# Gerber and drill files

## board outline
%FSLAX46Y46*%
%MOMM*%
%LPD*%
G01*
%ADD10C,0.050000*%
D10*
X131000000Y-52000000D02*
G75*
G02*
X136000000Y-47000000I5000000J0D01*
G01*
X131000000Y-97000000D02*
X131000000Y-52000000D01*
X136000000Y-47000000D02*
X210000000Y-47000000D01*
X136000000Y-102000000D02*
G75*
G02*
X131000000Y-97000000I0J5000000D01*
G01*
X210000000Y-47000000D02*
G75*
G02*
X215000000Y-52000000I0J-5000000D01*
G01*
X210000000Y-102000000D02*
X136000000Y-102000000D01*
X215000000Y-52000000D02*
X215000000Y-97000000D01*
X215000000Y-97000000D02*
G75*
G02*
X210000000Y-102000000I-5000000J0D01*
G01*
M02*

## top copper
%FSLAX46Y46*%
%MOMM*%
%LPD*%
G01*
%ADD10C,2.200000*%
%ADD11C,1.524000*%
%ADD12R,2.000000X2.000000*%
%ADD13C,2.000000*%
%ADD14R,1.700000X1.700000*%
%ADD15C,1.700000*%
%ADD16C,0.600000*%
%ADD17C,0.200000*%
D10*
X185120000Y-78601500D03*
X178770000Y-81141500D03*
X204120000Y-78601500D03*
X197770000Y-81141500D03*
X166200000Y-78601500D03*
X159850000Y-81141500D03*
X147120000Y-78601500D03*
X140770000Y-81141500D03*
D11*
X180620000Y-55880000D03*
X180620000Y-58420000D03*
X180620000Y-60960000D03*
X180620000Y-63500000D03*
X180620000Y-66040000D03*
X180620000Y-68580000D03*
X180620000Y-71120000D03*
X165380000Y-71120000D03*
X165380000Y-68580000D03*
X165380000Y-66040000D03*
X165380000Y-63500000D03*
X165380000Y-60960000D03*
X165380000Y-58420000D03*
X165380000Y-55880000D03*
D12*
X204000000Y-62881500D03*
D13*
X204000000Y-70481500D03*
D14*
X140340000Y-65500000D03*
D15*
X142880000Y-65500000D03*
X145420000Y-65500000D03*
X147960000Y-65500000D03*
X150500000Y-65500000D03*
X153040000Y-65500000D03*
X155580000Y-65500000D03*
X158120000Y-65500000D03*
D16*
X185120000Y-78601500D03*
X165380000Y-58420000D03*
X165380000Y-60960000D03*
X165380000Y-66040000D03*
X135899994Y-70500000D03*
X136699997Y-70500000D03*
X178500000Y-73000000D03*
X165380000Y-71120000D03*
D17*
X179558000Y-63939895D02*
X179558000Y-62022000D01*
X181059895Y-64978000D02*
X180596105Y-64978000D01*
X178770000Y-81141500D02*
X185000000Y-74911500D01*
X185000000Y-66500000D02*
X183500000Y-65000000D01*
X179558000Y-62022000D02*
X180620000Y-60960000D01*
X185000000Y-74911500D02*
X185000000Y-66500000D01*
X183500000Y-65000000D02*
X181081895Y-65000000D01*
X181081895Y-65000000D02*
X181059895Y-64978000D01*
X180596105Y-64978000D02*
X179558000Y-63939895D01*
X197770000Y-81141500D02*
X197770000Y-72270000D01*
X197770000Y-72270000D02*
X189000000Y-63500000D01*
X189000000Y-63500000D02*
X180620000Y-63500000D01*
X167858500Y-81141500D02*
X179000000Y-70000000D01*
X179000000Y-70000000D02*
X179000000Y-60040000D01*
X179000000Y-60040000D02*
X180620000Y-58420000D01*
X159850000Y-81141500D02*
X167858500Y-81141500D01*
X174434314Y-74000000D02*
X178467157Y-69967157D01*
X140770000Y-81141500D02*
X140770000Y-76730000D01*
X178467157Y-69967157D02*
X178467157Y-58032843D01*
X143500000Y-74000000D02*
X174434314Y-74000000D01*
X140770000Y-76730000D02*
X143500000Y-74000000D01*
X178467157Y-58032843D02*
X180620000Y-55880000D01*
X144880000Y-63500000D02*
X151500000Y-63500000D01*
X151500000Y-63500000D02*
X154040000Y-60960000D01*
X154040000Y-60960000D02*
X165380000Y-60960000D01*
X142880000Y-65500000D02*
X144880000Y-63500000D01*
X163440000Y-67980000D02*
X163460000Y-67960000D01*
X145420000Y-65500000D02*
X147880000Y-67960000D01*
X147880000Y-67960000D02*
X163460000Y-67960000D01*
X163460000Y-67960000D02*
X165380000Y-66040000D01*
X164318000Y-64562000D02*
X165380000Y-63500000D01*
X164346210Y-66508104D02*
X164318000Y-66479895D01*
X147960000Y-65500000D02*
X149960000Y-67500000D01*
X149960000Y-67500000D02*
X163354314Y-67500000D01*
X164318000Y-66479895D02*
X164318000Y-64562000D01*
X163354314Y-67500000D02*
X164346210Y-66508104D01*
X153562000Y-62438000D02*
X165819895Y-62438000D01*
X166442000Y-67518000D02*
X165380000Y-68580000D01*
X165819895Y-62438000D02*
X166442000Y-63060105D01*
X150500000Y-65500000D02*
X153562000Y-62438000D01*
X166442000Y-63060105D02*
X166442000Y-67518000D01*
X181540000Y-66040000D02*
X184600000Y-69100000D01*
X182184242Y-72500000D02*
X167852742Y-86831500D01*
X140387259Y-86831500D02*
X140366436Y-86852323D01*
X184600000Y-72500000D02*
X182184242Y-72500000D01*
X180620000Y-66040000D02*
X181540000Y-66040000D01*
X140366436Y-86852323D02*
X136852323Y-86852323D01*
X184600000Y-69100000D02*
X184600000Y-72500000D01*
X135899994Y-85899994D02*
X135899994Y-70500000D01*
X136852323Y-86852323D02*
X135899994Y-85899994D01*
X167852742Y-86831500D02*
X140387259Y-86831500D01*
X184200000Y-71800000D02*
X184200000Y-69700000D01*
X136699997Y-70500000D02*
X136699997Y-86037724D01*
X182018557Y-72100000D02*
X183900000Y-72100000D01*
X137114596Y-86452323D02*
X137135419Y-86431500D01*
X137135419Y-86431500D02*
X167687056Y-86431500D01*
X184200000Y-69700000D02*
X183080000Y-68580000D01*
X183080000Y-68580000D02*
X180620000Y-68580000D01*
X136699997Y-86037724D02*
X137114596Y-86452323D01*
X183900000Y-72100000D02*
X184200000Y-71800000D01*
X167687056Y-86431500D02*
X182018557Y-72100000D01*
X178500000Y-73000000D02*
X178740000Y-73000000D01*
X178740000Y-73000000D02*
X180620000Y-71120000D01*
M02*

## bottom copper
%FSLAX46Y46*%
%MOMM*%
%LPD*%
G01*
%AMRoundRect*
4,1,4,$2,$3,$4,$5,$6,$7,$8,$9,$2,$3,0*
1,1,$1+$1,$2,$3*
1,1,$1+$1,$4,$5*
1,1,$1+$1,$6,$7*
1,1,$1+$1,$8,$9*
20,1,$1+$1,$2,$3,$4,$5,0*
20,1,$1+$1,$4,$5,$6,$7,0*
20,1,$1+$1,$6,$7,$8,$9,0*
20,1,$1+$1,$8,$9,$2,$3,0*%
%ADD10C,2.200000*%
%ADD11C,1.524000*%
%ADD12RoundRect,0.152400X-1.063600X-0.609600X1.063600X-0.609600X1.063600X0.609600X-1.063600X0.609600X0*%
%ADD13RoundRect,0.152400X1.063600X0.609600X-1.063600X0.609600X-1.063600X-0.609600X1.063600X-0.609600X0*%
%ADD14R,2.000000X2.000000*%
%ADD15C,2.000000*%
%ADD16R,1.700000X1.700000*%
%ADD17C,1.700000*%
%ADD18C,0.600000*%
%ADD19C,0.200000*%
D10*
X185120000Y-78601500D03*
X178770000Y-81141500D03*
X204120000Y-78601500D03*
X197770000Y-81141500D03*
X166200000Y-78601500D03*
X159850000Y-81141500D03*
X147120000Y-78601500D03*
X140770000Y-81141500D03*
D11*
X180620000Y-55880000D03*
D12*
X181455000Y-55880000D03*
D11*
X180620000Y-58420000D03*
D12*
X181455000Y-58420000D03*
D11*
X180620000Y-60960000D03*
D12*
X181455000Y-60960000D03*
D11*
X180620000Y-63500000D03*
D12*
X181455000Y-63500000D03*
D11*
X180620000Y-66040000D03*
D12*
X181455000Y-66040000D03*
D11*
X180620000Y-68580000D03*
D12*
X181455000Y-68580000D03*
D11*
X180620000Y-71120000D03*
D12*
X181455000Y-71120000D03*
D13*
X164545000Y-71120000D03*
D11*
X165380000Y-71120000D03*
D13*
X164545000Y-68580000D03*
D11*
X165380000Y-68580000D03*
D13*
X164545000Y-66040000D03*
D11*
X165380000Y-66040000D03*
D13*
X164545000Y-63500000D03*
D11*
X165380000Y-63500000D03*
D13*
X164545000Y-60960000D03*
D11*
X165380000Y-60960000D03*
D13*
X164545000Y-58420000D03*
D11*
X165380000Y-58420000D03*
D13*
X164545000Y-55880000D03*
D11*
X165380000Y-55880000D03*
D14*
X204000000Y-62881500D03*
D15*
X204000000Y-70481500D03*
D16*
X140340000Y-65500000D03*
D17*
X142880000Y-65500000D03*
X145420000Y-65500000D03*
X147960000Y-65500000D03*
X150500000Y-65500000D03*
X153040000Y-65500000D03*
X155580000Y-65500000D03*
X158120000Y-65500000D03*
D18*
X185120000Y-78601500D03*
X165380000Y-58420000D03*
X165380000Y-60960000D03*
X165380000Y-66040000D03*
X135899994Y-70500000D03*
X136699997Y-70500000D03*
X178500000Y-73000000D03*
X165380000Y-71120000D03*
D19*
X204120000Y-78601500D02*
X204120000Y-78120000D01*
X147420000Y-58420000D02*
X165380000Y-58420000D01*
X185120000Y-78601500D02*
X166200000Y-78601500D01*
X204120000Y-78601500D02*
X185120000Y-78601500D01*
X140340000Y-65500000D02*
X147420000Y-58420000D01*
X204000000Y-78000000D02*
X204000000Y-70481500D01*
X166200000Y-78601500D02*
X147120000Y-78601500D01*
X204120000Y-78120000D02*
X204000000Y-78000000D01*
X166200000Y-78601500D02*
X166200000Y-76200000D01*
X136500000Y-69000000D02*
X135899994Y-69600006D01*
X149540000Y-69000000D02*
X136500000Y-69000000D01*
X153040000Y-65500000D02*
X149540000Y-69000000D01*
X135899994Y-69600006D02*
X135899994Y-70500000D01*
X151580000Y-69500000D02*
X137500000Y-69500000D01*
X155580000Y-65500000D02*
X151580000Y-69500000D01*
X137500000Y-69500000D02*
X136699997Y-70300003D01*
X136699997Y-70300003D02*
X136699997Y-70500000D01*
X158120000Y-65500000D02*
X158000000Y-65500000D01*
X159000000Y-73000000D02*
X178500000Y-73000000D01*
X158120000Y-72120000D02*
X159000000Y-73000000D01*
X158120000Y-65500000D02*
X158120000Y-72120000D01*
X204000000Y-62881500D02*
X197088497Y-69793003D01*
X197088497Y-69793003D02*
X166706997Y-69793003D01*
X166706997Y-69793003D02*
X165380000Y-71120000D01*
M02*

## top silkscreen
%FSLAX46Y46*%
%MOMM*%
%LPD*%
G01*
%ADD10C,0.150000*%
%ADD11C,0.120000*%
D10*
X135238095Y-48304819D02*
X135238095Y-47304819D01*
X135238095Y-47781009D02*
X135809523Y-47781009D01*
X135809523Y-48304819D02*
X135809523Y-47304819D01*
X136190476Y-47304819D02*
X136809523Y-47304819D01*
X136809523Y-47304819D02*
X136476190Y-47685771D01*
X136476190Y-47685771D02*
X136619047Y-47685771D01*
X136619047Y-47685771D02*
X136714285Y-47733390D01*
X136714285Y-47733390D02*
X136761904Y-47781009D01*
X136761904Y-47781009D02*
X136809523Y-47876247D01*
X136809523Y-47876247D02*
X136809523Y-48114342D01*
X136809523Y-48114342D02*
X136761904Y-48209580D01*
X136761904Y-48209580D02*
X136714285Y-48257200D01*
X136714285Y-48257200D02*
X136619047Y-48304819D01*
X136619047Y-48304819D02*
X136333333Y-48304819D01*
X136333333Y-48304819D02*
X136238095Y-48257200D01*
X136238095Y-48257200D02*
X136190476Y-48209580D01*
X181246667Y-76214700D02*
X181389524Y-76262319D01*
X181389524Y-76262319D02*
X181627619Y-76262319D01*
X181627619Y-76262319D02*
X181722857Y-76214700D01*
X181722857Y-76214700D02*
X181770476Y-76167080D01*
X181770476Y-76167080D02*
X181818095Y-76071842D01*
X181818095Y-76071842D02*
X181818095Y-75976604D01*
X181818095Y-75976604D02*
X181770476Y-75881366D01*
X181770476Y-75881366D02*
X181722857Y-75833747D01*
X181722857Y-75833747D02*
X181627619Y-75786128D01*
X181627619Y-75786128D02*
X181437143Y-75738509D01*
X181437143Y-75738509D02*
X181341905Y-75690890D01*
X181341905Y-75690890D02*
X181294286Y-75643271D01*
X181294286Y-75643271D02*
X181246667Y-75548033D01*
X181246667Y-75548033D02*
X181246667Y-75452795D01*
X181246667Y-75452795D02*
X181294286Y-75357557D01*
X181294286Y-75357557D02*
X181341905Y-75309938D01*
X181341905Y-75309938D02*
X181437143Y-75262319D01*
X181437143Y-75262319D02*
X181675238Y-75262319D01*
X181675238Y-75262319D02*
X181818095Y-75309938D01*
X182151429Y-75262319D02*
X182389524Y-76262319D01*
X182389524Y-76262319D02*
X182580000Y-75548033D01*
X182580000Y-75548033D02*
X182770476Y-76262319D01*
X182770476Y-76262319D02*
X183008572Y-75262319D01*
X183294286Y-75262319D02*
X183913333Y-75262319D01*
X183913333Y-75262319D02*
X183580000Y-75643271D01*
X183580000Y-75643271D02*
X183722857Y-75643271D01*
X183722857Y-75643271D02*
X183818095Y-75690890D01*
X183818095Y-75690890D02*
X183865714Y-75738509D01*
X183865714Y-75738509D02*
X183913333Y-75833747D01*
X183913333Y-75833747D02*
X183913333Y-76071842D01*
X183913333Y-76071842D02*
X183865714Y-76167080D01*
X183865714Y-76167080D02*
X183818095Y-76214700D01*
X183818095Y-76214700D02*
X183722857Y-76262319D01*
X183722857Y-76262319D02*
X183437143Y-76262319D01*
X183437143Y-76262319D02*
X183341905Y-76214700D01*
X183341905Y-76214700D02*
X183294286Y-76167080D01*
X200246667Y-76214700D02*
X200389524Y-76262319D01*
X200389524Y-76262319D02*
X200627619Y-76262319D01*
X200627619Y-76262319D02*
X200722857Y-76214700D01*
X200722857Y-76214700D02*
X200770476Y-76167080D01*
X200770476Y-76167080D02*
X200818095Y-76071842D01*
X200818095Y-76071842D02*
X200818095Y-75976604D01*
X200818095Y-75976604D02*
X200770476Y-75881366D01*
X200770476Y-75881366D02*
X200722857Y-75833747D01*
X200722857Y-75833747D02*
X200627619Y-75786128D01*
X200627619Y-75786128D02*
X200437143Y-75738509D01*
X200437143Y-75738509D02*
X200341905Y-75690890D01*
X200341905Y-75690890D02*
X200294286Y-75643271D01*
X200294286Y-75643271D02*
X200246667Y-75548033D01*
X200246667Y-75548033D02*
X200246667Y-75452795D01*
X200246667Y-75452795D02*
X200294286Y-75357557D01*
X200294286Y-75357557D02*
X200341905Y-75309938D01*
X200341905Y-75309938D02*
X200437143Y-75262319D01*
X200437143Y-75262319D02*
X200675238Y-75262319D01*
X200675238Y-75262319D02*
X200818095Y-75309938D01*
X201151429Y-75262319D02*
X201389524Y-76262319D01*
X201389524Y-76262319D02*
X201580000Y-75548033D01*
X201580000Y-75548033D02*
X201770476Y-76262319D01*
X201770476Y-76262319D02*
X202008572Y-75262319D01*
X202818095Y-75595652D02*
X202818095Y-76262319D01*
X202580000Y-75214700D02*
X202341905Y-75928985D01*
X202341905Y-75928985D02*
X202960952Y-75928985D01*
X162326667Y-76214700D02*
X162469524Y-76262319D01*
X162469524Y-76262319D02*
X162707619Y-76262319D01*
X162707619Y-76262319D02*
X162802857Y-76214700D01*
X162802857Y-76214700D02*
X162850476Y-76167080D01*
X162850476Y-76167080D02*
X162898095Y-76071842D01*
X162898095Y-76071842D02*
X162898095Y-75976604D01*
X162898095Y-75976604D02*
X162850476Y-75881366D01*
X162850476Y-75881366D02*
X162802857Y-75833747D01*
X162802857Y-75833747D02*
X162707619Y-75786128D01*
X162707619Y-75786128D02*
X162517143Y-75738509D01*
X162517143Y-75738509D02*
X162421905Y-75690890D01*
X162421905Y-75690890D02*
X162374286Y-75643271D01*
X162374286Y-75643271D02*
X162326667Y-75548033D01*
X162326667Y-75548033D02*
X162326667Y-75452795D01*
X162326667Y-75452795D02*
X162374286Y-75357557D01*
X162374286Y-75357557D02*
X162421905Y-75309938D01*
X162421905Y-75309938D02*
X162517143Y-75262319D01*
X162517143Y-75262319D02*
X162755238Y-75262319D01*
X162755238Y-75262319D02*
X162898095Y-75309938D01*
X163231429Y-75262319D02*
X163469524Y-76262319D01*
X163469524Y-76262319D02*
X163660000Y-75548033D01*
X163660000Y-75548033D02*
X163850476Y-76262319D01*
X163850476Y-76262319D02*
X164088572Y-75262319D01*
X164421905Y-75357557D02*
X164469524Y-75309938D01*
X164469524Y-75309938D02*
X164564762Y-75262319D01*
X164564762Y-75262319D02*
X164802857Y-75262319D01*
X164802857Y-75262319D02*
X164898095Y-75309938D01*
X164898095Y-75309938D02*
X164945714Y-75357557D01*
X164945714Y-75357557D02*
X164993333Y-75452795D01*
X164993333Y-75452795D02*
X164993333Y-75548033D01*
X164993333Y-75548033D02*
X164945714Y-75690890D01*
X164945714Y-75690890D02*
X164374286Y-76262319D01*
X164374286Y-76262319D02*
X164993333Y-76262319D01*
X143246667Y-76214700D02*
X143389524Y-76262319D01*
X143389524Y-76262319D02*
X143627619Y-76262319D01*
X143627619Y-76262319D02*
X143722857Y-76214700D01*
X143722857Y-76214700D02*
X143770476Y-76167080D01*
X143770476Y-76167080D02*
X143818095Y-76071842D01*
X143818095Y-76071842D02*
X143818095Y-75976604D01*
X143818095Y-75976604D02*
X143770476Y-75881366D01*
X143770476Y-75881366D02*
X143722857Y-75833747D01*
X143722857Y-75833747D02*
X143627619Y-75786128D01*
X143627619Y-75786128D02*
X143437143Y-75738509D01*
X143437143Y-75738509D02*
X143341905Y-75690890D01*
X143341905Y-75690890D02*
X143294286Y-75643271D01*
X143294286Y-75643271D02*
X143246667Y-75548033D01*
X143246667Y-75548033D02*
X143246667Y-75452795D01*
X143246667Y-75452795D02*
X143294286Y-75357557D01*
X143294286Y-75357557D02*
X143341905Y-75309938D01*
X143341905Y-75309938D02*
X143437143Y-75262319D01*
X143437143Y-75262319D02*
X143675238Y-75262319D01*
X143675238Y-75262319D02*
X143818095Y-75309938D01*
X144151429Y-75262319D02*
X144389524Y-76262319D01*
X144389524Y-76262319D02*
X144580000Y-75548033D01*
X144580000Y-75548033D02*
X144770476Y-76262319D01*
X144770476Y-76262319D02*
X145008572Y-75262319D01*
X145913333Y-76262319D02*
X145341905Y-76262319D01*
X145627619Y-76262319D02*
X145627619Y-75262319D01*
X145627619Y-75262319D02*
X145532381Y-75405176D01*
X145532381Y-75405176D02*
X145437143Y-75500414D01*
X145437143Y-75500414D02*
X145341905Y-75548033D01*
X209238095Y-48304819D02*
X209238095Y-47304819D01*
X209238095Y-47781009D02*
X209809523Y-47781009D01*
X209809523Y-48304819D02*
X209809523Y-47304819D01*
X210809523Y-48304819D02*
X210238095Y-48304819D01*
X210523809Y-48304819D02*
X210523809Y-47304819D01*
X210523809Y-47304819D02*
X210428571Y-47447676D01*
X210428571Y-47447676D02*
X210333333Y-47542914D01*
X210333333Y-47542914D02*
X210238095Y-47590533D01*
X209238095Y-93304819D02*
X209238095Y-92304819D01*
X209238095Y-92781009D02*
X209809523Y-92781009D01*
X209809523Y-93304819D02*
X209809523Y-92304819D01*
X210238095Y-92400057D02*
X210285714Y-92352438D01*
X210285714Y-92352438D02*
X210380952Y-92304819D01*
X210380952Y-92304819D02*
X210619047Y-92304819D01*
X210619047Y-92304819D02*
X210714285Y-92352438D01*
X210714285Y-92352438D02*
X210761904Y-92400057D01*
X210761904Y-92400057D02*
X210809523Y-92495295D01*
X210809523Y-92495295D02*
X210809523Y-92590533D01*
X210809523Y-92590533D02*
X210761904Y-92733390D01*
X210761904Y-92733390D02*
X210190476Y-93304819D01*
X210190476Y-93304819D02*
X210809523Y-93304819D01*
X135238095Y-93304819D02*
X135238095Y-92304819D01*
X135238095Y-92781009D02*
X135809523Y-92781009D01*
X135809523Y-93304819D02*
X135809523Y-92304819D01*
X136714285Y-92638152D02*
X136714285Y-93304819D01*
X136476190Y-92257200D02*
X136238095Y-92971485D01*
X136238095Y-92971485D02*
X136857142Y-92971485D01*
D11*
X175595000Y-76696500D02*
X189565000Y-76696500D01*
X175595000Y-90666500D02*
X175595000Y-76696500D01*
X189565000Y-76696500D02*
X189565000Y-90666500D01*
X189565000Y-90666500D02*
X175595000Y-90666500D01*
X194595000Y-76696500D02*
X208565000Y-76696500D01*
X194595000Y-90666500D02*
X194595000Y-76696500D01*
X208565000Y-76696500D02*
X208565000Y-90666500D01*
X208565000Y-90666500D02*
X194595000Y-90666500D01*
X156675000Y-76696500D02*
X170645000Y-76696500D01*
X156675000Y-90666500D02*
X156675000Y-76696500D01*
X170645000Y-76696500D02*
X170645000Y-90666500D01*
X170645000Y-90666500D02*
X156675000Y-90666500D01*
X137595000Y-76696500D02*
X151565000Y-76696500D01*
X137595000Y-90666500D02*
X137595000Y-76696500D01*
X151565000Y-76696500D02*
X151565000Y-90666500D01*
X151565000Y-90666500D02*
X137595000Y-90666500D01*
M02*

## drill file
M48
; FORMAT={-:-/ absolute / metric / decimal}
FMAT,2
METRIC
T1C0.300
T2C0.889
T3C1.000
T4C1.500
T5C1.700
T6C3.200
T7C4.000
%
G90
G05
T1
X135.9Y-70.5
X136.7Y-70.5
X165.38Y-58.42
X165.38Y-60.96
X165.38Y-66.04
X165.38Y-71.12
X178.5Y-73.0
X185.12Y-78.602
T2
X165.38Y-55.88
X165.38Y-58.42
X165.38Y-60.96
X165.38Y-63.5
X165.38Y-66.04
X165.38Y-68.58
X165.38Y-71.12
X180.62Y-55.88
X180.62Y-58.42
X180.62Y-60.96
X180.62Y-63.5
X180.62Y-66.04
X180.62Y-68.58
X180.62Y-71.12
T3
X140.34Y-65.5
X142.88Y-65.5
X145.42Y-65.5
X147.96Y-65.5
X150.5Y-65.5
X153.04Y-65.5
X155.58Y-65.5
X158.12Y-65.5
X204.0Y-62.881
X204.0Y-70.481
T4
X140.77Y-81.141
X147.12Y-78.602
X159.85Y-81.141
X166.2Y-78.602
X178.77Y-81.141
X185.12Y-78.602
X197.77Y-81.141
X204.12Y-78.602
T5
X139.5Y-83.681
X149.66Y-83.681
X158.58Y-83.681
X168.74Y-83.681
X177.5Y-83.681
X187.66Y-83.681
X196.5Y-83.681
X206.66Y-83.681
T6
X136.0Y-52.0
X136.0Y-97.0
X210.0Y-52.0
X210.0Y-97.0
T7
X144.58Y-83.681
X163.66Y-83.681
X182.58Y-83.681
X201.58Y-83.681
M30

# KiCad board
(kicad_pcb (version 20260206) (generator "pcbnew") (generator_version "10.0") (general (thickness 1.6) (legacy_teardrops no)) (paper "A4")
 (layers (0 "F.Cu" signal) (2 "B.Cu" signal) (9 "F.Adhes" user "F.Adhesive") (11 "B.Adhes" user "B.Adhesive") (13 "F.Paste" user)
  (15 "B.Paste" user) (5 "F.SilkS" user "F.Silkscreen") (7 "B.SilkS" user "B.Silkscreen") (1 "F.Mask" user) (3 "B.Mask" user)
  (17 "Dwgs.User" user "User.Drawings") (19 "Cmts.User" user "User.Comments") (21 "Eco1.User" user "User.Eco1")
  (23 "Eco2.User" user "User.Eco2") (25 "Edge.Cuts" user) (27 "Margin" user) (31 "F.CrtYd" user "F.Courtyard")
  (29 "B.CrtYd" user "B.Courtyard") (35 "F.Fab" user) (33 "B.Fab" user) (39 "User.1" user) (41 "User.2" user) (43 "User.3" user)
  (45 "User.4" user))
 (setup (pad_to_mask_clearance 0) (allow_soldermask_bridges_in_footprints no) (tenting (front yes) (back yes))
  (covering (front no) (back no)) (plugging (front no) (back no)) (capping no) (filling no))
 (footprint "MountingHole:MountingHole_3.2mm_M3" (layer "F.Cu") (at 136 52)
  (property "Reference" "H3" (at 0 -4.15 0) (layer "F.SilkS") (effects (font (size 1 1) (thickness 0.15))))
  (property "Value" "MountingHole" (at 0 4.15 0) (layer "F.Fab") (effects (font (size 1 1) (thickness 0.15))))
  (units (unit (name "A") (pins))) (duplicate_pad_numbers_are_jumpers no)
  (pad "" np_thru_hole circle (at 0 0) (size 3.2 3.2) (drill 3.2) (layers "*.Cu" "*.Mask")))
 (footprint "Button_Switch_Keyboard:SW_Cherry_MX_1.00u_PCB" (layer "F.Cu") (at 185.12 78.6015)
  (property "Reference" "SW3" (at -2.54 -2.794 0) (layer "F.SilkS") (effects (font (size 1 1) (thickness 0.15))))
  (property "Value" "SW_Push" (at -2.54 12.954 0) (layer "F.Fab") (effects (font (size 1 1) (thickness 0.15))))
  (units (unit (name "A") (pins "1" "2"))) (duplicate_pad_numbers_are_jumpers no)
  (fp_line (start -9.525 -1.905) (end 4.445 -1.905) (stroke (width 0.12) (type solid)) (layer "F.SilkS"))
  (fp_line (start -9.525 12.065) (end -9.525 -1.905) (stroke (width 0.12) (type solid)) (layer "F.SilkS"))
  (fp_line (start 4.445 -1.905) (end 4.445 12.065) (stroke (width 0.12) (type solid)) (layer "F.SilkS"))
  (fp_line (start 4.445 12.065) (end -9.525 12.065) (stroke (width 0.12) (type solid)) (layer "F.SilkS"))
  (pad "" np_thru_hole circle (at -7.62 5.08) (size 1.7 1.7) (drill 1.7) (layers "*.Cu" "*.Mask"))
  (pad "" np_thru_hole circle (at -2.54 5.08) (size 4 4) (drill 4) (layers "*.Cu" "*.Mask"))
  (pad "" np_thru_hole circle (at 2.54 5.08) (size 1.7 1.7) (drill 1.7) (layers "*.Cu" "*.Mask"))
  (pad "1" thru_hole circle (at 0 0) (size 2.2 2.2) (drill 1.5) (layers "*.Cu" "*.Mask") (remove_unused_layers no) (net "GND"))
  (pad "2" thru_hole circle (at -6.35 2.54) (size 2.2 2.2) (drill 1.5) (layers "*.Cu" "*.Mask") (remove_unused_layers no)
   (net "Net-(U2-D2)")))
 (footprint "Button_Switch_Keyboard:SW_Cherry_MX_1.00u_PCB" (layer "F.Cu") (at 204.12 78.6015)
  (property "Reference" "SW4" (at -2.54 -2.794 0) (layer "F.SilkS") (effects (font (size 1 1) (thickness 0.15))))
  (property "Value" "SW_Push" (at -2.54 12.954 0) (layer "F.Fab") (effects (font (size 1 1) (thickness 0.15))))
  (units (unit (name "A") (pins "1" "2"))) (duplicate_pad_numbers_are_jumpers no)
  (fp_line (start -9.525 -1.905) (end 4.445 -1.905) (stroke (width 0.12) (type solid)) (layer "F.SilkS"))
  (fp_line (start -9.525 12.065) (end -9.525 -1.905) (stroke (width 0.12) (type solid)) (layer "F.SilkS"))
  (fp_line (start 4.445 -1.905) (end 4.445 12.065) (stroke (width 0.12) (type solid)) (layer "F.SilkS"))
  (fp_line (start 4.445 12.065) (end -9.525 12.065) (stroke (width 0.12) (type solid)) (layer "F.SilkS"))
  (pad "" np_thru_hole circle (at -7.62 5.08) (size 1.7 1.7) (drill 1.7) (layers "*.Cu" "*.Mask"))
  (pad "" np_thru_hole circle (at -2.54 5.08) (size 4 4) (drill 4) (layers "*.Cu" "*.Mask"))
  (pad "" np_thru_hole circle (at 2.54 5.08) (size 1.7 1.7) (drill 1.7) (layers "*.Cu" "*.Mask"))
  (pad "1" thru_hole circle (at 0 0) (size 2.2 2.2) (drill 1.5) (layers "*.Cu" "*.Mask") (remove_unused_layers no) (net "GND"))
  (pad "2" thru_hole circle (at -6.35 2.54) (size 2.2 2.2) (drill 1.5) (layers "*.Cu" "*.Mask") (remove_unused_layers no)
   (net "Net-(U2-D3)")))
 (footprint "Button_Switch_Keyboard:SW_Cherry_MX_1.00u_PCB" (layer "F.Cu") (at 166.2 78.6015)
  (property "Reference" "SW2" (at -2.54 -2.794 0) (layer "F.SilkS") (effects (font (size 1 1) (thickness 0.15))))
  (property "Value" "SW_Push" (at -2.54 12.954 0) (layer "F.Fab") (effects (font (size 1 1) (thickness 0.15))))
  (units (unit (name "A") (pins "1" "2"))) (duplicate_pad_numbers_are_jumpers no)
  (fp_line (start -9.525 -1.905) (end 4.445 -1.905) (stroke (width 0.12) (type solid)) (layer "F.SilkS"))
  (fp_line (start -9.525 12.065) (end -9.525 -1.905) (stroke (width 0.12) (type solid)) (layer "F.SilkS"))
  (fp_line (start 4.445 -1.905) (end 4.445 12.065) (stroke (width 0.12) (type solid)) (layer "F.SilkS"))
  (fp_line (start 4.445 12.065) (end -9.525 12.065) (stroke (width 0.12) (type solid)) (layer "F.SilkS"))
  (pad "" np_thru_hole circle (at -7.62 5.08) (size 1.7 1.7) (drill 1.7) (layers "*.Cu" "*.Mask"))
  (pad "" np_thru_hole circle (at -2.54 5.08) (size 4 4) (drill 4) (layers "*.Cu" "*.Mask"))
  (pad "" np_thru_hole circle (at 2.54 5.08) (size 1.7 1.7) (drill 1.7) (layers "*.Cu" "*.Mask"))
  (pad "1" thru_hole circle (at 0 0) (size 2.2 2.2) (drill 1.5) (layers "*.Cu" "*.Mask") (remove_unused_layers no) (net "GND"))
  (pad "2" thru_hole circle (at -6.35 2.54) (size 2.2 2.2) (drill 1.5) (layers "*.Cu" "*.Mask") (remove_unused_layers no)
   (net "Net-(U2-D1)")))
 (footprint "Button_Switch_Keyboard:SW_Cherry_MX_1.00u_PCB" (layer "F.Cu") (at 147.12 78.6015)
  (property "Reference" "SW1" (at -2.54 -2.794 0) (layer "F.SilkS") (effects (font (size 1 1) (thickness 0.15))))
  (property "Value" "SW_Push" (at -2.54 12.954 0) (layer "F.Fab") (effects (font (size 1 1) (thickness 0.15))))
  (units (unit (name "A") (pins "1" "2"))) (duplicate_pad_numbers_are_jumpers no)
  (fp_line (start -9.525 -1.905) (end 4.445 -1.905) (stroke (width 0.12) (type solid)) (layer "F.SilkS"))
  (fp_line (start -9.525 12.065) (end -9.525 -1.905) (stroke (width 0.12) (type solid)) (layer "F.SilkS"))
  (fp_line (start 4.445 -1.905) (end 4.445 12.065) (stroke (width 0.12) (type solid)) (layer "F.SilkS"))
  (fp_line (start 4.445 12.065) (end -9.525 12.065) (stroke (width 0.12) (type solid)) (layer "F.SilkS"))
  (pad "" np_thru_hole circle (at -7.62 5.08) (size 1.7 1.7) (drill 1.7) (layers "*.Cu" "*.Mask"))
  (pad "" np_thru_hole circle (at -2.54 5.08) (size 4 4) (drill 4) (layers "*.Cu" "*.Mask"))
  (pad "" np_thru_hole circle (at 2.54 5.08) (size 1.7 1.7) (drill 1.7) (layers "*.Cu" "*.Mask"))
  (pad "1" thru_hole circle (at 0 0) (size 2.2 2.2) (drill 1.5) (layers "*.Cu" "*.Mask") (remove_unused_layers no) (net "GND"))
  (pad "2" thru_hole circle (at -6.35 2.54) (size 2.2 2.2) (drill 1.5) (layers "*.Cu" "*.Mask") (remove_unused_layers no)
   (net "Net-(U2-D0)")))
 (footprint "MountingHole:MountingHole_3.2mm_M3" (layer "F.Cu") (at 210 52)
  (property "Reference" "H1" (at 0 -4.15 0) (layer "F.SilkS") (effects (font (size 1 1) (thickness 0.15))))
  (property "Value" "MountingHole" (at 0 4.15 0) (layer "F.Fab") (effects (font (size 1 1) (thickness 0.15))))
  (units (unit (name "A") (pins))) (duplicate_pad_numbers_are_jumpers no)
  (pad "" np_thru_hole circle (at 0 0) (size 3.2 3.2) (drill 3.2) (layers "*.Cu" "*.Mask")))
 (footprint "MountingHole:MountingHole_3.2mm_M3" (layer "F.Cu") (at 210 97)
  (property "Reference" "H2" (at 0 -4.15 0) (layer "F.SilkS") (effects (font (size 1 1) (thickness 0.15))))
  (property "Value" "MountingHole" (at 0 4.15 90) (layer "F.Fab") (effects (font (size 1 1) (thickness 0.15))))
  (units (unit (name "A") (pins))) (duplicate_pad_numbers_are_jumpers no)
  (pad "" np_thru_hole circle (at 0 0) (size 3.2 3.2) (drill 3.2) (layers "*.Cu" "*.Mask")))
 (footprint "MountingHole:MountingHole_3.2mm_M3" (layer "F.Cu") (at 136 97)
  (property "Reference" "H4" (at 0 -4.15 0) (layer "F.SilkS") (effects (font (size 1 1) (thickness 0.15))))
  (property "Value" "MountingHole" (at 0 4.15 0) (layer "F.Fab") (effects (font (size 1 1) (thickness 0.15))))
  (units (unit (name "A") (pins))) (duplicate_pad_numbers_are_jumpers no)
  (pad "" np_thru_hole circle (at 0 0) (size 3.2 3.2) (drill 3.2) (layers "*.Cu" "*.Mask")))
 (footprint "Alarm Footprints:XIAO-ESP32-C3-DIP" (layer "B.Cu") (at 173 63.5 90)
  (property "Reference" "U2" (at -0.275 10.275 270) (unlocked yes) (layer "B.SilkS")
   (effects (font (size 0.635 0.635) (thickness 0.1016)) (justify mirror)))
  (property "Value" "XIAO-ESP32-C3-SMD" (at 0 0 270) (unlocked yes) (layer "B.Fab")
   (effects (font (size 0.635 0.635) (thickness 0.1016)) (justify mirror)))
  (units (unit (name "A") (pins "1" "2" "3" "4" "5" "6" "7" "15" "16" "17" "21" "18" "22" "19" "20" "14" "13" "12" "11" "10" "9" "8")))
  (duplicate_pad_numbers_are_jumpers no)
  (pad "1" thru_hole circle (at 7.62 7.62) (size 1.524 1.524) (drill 0.889) (layers "*.Cu" "*.Mask") (remove_unused_layers no)
   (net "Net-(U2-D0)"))
  (pad "1" smd roundrect (at 7.62 8.455) (size 2.432 1.524) (layers "B.Cu" "B.Mask") (roundrect_rratio 0.1) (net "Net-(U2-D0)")
   (thermal_bridge_angle 45))
  (pad "2" thru_hole circle (at 5.08 7.62) (size 1.524 1.524) (drill 0.889) (layers "*.Cu" "*.Mask") (remove_unused_layers no)
   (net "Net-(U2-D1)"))
  (pad "2" smd roundrect (at 5.08 8.455) (size 2.432 1.524) (layers "B.Cu" "B.Mask") (roundrect_rratio 0.1) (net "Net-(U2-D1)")
   (thermal_bridge_angle 45))
  (pad "3" thru_hole circle (at 2.54 7.62) (size 1.524 1.524) (drill 0.889) (layers "*.Cu" "*.Mask") (remove_unused_layers no)
   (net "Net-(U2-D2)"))
  (pad "3" smd roundrect (at 2.54 8.455) (size 2.432 1.524) (layers "B.Cu" "B.Mask") (roundrect_rratio 0.1) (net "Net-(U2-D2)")
   (thermal_bridge_angle 45))
  (pad "4" thru_hole circle (at 0 7.62) (size 1.524 1.524) (drill 0.889) (layers "*.Cu" "*.Mask") (remove_unused_layers no)
   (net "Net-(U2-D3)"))
  (pad "4" smd roundrect (at 0 8.455) (size 2.432 1.524) (layers "B.Cu" "B.Mask") (roundrect_rratio 0.1) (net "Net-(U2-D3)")
   (thermal_bridge_angle 45))
  (pad "5" thru_hole circle (at -2.54 7.62) (size 1.524 1.524) (drill 0.889) (layers "*.Cu" "*.Mask") (remove_unused_layers no) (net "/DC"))
  (pad "5" smd roundrect (at -2.54 8.455) (size 2.432 1.524) (layers "B.Cu" "B.Mask") (roundrect_rratio 0.1) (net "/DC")
   (thermal_bridge_angle 45))
  (pad "6" thru_hole circle (at -5.08 7.62) (size 1.524 1.524) (drill 0.889) (layers "*.Cu" "*.Mask") (remove_unused_layers no) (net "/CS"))
  (pad "6" smd roundrect (at -5.08 8.455) (size 2.432 1.524) (layers "B.Cu" "B.Mask") (roundrect_rratio 0.1) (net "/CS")
   (thermal_bridge_angle 45))
  (pad "7" thru_hole circle (at -7.62 7.62) (size 1.524 1.524) (drill 0.889) (layers "*.Cu" "*.Mask") (remove_unused_layers no) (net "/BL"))
  (pad "7" smd roundrect (at -7.62 8.455) (size 2.432 1.524) (layers "B.Cu" "B.Mask") (roundrect_rratio 0.1) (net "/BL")
   (thermal_bridge_angle 45))
  (pad "8" smd roundrect (at -7.62 -8.455 180) (size 2.432 1.524) (layers "B.Cu" "B.Mask") (roundrect_rratio 0.1) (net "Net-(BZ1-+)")
   (thermal_bridge_angle 45))
  (pad "8" thru_hole circle (at -7.62 -7.62 180) (size 1.524 1.524) (drill 0.889) (layers "*.Cu" "*.Mask") (remove_unused_layers no)
   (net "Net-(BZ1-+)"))
  (pad "9" smd roundrect (at -5.08 -8.455 180) (size 2.432 1.524) (layers "B.Cu" "B.Mask") (roundrect_rratio 0.1) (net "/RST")
   (thermal_bridge_angle 45))
  (pad "9" thru_hole circle (at -5.08 -7.62 180) (size 1.524 1.524) (drill 0.889) (layers "*.Cu" "*.Mask") (remove_unused_layers no)
   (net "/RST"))
  (pad "10" smd roundrect (at -2.54 -8.455 180) (size 2.432 1.524) (layers "B.Cu" "B.Mask") (roundrect_rratio 0.1) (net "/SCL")
   (thermal_bridge_angle 45))
  (pad "10" thru_hole circle (at -2.54 -7.62 180) (size 1.524 1.524) (drill 0.889) (layers "*.Cu" "*.Mask") (remove_unused_layers no)
   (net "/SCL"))
  (pad "11" smd roundrect (at 0 -8.455 180) (size 2.432 1.524) (layers "B.Cu" "B.Mask") (roundrect_rratio 0.1) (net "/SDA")
   (thermal_bridge_angle 45))
  (pad "11" thru_hole circle (at 0 -7.62 180) (size 1.524 1.524) (drill 0.889) (layers "*.Cu" "*.Mask") (remove_unused_layers no)
   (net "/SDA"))
  (pad "12" smd roundrect (at 2.54 -8.455 180) (size 2.432 1.524) (layers "B.Cu" "B.Mask") (roundrect_rratio 0.1) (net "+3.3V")
   (thermal_bridge_angle 45))
  (pad "12" thru_hole circle (at 2.54 -7.62 180) (size 1.524 1.524) (drill 0.889) (layers "*.Cu" "*.Mask") (remove_unused_layers no)
   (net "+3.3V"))
  (pad "13" smd roundrect (at 5.08 -8.455 180) (size 2.432 1.524) (layers "B.Cu" "B.Mask") (roundrect_rratio 0.1) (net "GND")
   (thermal_bridge_angle 45))
  (pad "13" thru_hole circle (at 5.08 -7.62 180) (size 1.524 1.524) (drill 0.889) (layers "*.Cu" "*.Mask") (remove_unused_layers no)
   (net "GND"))
  (pad "14" smd roundrect (at 7.62 -8.455 180) (size 2.432 1.524) (layers "B.Cu" "B.Mask") (roundrect_rratio 0.1)
   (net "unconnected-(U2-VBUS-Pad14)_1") (thermal_bridge_angle 45))
  (pad "14" thru_hole circle (at 7.62 -7.62 180) (size 1.524 1.524) (drill 0.889) (layers "*.Cu" "*.Mask") (remove_unused_layers no)
   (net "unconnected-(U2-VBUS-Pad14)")))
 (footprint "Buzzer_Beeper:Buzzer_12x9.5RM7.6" (layer "B.Cu") (at 204 62.8815 -90)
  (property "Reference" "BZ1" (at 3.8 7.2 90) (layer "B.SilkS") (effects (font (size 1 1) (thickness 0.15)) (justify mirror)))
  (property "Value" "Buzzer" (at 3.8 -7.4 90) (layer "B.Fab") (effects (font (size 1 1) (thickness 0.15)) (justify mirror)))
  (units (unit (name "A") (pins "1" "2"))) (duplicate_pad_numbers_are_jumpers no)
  (pad "1" thru_hole rect (at 0 0 270) (size 2 2) (drill 1) (layers "*.Cu" "*.Mask") (remove_unused_layers no) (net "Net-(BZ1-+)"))
  (pad "2" thru_hole circle (at 7.6 0 270) (size 2 2) (drill 1) (layers "*.Cu" "*.Mask") (remove_unused_layers no) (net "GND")))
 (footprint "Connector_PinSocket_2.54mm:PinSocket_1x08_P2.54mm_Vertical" (layer "B.Cu") (at 140.34 65.5 -90)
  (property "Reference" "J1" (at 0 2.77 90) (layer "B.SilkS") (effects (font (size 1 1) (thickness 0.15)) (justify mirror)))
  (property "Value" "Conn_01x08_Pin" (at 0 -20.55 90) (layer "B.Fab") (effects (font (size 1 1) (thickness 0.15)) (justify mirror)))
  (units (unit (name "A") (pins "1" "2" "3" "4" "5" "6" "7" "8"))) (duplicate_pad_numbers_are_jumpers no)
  (pad "1" thru_hole rect (at 0 0 270) (size 1.7 1.7) (drill 1) (layers "*.Cu" "*.Mask") (remove_unused_layers no) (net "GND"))
  (pad "2" thru_hole circle (at 0 -2.54 270) (size 1.7 1.7) (drill 1) (layers "*.Cu" "*.Mask") (remove_unused_layers no) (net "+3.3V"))
  (pad "3" thru_hole circle (at 0 -5.08 270) (size 1.7 1.7) (drill 1) (layers "*.Cu" "*.Mask") (remove_unused_layers no) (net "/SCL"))
  (pad "4" thru_hole circle (at 0 -7.62 270) (size 1.7 1.7) (drill 1) (layers "*.Cu" "*.Mask") (remove_unused_layers no) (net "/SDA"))
  (pad "5" thru_hole circle (at 0 -10.16 270) (size 1.7 1.7) (drill 1) (layers "*.Cu" "*.Mask") (remove_unused_layers no) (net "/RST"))
  (pad "6" thru_hole circle (at 0 -12.7 270) (size 1.7 1.7) (drill 1) (layers "*.Cu" "*.Mask") (remove_unused_layers no) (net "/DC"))
  (pad "7" thru_hole circle (at 0 -15.24 270) (size 1.7 1.7) (drill 1) (layers "*.Cu" "*.Mask") (remove_unused_layers no) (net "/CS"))
  (pad "8" thru_hole circle (at 0 -17.78 270) (size 1.7 1.7) (drill 1) (layers "*.Cu" "*.Mask") (remove_unused_layers no) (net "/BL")))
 (gr_arc (start 131 52) (mid 132.464466 48.464466) (end 136 47) (stroke (width 0.05) (type default)) (layer "Edge.Cuts"))
 (gr_line (start 131 97) (end 131 52) (stroke (width 0.05) (type default)) (layer "Edge.Cuts"))
 (gr_line (start 136 47) (end 210 47) (stroke (width 0.05) (type default)) (layer "Edge.Cuts"))
 (gr_arc (start 136 102) (mid 132.464466 100.535534) (end 131 97) (stroke (width 0.05) (type default)) (layer "Edge.Cuts"))
 (gr_arc (start 210 47) (mid 213.535534 48.464466) (end 215 52) (stroke (width 0.05) (type default)) (layer "Edge.Cuts"))
 (gr_line (start 210 102) (end 136 102) (stroke (width 0.05) (type default)) (layer "Edge.Cuts"))
 (gr_line (start 215 52) (end 215 97) (stroke (width 0.05) (type default)) (layer "Edge.Cuts"))
 (gr_arc (start 215 97) (mid 213.535534 100.535534) (end 210 102) (stroke (width 0.05) (type default)) (layer "Edge.Cuts"))
 (via (at 185.12 78.6015) (size 0.6) (drill 0.3) (layers "F.Cu" "B.Cu") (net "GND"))
 (via (at 165.38 58.42) (size 0.6) (drill 0.3) (layers "F.Cu" "B.Cu") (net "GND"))
 (segment (start 204.12 78.6015) (end 204.12 78.12) (width 0.2) (layer "B.Cu") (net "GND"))
 (segment (start 147.42 58.42) (end 165.38 58.42) (width 0.2) (layer "B.Cu") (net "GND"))
 (segment (start 185.12 78.6015) (end 166.2 78.6015) (width 0.2) (layer "B.Cu") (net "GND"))
 (segment (start 204.12 78.6015) (end 185.12 78.6015) (width 0.2) (layer "B.Cu") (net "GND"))
 (segment (start 140.34 65.5) (end 147.42 58.42) (width 0.2) (layer "B.Cu") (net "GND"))
 (segment (start 204 78) (end 204 70.4815) (width 0.2) (layer "B.Cu") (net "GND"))
 (segment (start 166.2 78.6015) (end 147.12 78.6015) (width 0.2) (layer "B.Cu") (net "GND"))
 (segment (start 204.12 78.12) (end 204 78) (width 0.2) (layer "B.Cu") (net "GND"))
 (segment (start 166.2 78.6015) (end 166.2 76.2) (width 0.2) (layer "B.Cu") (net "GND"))
 (segment (start 179.558 63.939895) (end 179.558 62.022) (width 0.2) (layer "F.Cu") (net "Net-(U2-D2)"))
 (segment (start 181.059895 64.978) (end 180.596105 64.978) (width 0.2) (layer "F.Cu") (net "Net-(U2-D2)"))
 (segment (start 178.77 81.1415) (end 185 74.9115) (width 0.2) (layer "F.Cu") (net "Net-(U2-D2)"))
 (segment (start 185 66.5) (end 183.5 65) (width 0.2) (layer "F.Cu") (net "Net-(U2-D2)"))
 (segment (start 179.558 62.022) (end 180.62 60.96) (width 0.2) (layer "F.Cu") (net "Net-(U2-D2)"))
 (segment (start 185 74.9115) (end 185 66.5) (width 0.2) (layer "F.Cu") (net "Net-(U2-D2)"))
 (segment (start 183.5 65) (end 181.081895 65) (width 0.2) (layer "F.Cu") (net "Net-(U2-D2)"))
 (segment (start 181.081895 65) (end 181.059895 64.978) (width 0.2) (layer "F.Cu") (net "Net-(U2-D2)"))
 (segment (start 180.596105 64.978) (end 179.558 63.939895) (width 0.2) (layer "F.Cu") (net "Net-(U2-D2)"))
 (segment (start 197.77 81.1415) (end 197.77 72.27) (width 0.2) (layer "F.Cu") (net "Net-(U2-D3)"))
 (segment (start 197.77 72.27) (end 189 63.5) (width 0.2) (layer "F.Cu") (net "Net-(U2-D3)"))
 (segment (start 189 63.5) (end 180.62 63.5) (width 0.2) (layer "F.Cu") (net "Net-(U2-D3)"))
 (segment (start 167.8585 81.1415) (end 179 70) (width 0.2) (layer "F.Cu") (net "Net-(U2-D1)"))
 (segment (start 179 70) (end 179 60.04) (width 0.2) (layer "F.Cu") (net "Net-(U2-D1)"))
 (segment (start 179 60.04) (end 180.62 58.42) (width 0.2) (layer "F.Cu") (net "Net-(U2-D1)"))
 (segment (start 159.85 81.1415) (end 167.8585 81.1415) (width 0.2) (layer "F.Cu") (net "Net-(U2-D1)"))
 (segment (start 174.434314 74) (end 178.467157 69.967157) (width 0.2) (layer "F.Cu") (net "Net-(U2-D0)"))
 (segment (start 140.77 81.1415) (end 140.77 76.73) (width 0.2) (layer "F.Cu") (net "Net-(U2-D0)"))
 (segment (start 178.467157 69.967157) (end 178.467157 58.032843) (width 0.2) (layer "F.Cu") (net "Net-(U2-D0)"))
 (segment (start 143.5 74) (end 174.434314 74) (width 0.2) (layer "F.Cu") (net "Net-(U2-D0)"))
 (segment (start 140.77 76.73) (end 143.5 74) (width 0.2) (layer "F.Cu") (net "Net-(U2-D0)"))
 (segment (start 178.467157 58.032843) (end 180.62 55.88) (width 0.2) (layer "F.Cu") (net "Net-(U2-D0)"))
 (segment (start 144.88 63.5) (end 151.5 63.5) (width 0.2) (layer "F.Cu") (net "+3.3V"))
 (segment (start 151.5 63.5) (end 154.04 60.96) (width 0.2) (layer "F.Cu") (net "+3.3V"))
 (segment (start 154.04 60.96) (end 165.38 60.96) (width 0.2) (layer "F.Cu") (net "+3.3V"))
 (segment (start 142.88 65.5) (end 144.88 63.5) (width 0.2) (layer "F.Cu") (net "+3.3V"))
 (via (at 165.38 60.96) (size 0.6) (drill 0.3) (layers "F.Cu" "B.Cu") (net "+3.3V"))
 (segment (start 163.44 67.98) (end 163.46 67.96) (width 0.2) (layer "F.Cu") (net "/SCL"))
 (segment (start 145.42 65.5) (end 147.88 67.96) (width 0.2) (layer "F.Cu") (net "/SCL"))
 (segment (start 147.88 67.96) (end 163.46 67.96) (width 0.2) (layer "F.Cu") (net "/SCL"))
 (segment (start 163.46 67.96) (end 165.38 66.04) (width 0.2) (layer "F.Cu") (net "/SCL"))
 (via (at 165.38 66.04) (size 0.6) (drill 0.3) (layers "F.Cu" "B.Cu") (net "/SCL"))
 (segment (start 164.318 64.562) (end 165.38 63.5) (width 0.2) (layer "F.Cu") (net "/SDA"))
 (segment (start 164.34621 66.508104) (end 164.318 66.479895) (width 0.2) (layer "F.Cu") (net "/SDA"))
 (segment (start 147.96 65.5) (end 149.96 67.5) (width 0.2) (layer "F.Cu") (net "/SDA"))
 (segment (start 149.96 67.5) (end 163.354314 67.5) (width 0.2) (layer "F.Cu") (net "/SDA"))
 (segment (start 164.318 66.479895) (end 164.318 64.562) (width 0.2) (layer "F.Cu") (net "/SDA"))
 (segment (start 163.354314 67.5) (end 164.34621 66.508104) (width 0.2) (layer "F.Cu") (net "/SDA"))
 (segment (start 153.562 62.438) (end 165.819895 62.438) (width 0.2) (layer "F.Cu") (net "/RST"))
 (segment (start 166.442 67.518) (end 165.38 68.58) (width 0.2) (layer "F.Cu") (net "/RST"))
 (segment (start 165.819895 62.438) (end 166.442 63.060105) (width 0.2) (layer "F.Cu") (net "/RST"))
 (segment (start 150.5 65.5) (end 153.562 62.438) (width 0.2) (layer "F.Cu") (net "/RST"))
 (segment (start 166.442 63.060105) (end 166.442 67.518) (width 0.2) (layer "F.Cu") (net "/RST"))
 (segment (start 181.54 66.04) (end 184.6 69.1) (width 0.2) (layer "F.Cu") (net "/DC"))
 (segment (start 182.184242 72.5) (end 167.852742 86.8315) (width 0.2) (layer "F.Cu") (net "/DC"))
 (segment (start 140.387259 86.8315) (end 140.366436 86.852323) (width 0.2) (layer "F.Cu") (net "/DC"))
 (segment (start 184.6 72.5) (end 182.184242 72.5) (width 0.2) (layer "F.Cu") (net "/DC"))
 (segment (start 180.62 66.04) (end 181.54 66.04) (width 0.2) (layer "F.Cu") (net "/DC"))
 (segment (start 140.366436 86.852323) (end 136.852323 86.852323) (width 0.2) (layer "F.Cu") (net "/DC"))
 (segment (start 184.6 69.1) (end 184.6 72.5) (width 0.2) (layer "F.Cu") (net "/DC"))
 (segment (start 135.899994 85.899994) (end 135.899994 70.5) (width 0.2) (layer "F.Cu") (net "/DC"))
 (segment (start 136.852323 86.852323) (end 135.899994 85.899994) (width 0.2) (layer "F.Cu") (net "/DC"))
 (segment (start 167.852742 86.8315) (end 140.387259 86.8315) (width 0.2) (layer "F.Cu") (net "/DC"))
 (via (at 135.899994 70.5) (size 0.6) (drill 0.3) (layers "F.Cu" "B.Cu") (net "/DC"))
 (segment (start 136.5 69) (end 135.899994 69.600006) (width 0.2) (layer "B.Cu") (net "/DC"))
 (segment (start 149.54 69) (end 136.5 69) (width 0.2) (layer "B.Cu") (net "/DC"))
 (segment (start 153.04 65.5) (end 149.54 69) (width 0.2) (layer "B.Cu") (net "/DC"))
 (segment (start 135.899994 69.600006) (end 135.899994 70.5) (width 0.2) (layer "B.Cu") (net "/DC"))
 (segment (start 184.2 71.8) (end 184.2 69.7) (width 0.2) (layer "F.Cu") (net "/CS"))
 (segment (start 136.699997 70.5) (end 136.699997 86.037724) (width 0.2) (layer "F.Cu") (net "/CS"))
 (segment (start 182.018557 72.1) (end 183.9 72.1) (width 0.2) (layer "F.Cu") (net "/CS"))
 (segment (start 137.114596 86.452323) (end 137.135419 86.4315) (width 0.2) (layer "F.Cu") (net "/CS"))
 (segment (start 137.135419 86.4315) (end 167.687056 86.4315) (width 0.2) (layer "F.Cu") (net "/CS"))
 (segment (start 184.2 69.7) (end 183.08 68.58) (width 0.2) (layer "F.Cu") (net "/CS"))
 (segment (start 183.08 68.58) (end 180.62 68.58) (width 0.2) (layer "F.Cu") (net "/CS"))
 (segment (start 136.699997 86.037724) (end 137.114596 86.452323) (width 0.2) (layer "F.Cu") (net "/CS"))
 (segment (start 183.9 72.1) (end 184.2 71.8) (width 0.2) (layer "F.Cu") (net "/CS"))
 (segment (start 167.687056 86.4315) (end 182.018557 72.1) (width 0.2) (layer "F.Cu") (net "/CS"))
 (via (at 136.699997 70.5) (size 0.6) (drill 0.3) (layers "F.Cu" "B.Cu") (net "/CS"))
 (segment (start 151.58 69.5) (end 137.5 69.5) (width 0.2) (layer "B.Cu") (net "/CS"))
 (segment (start 155.58 65.5) (end 151.58 69.5) (width 0.2) (layer "B.Cu") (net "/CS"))
 (segment (start 137.5 69.5) (end 136.699997 70.300003) (width 0.2) (layer "B.Cu") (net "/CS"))
 (segment (start 136.699997 70.300003) (end 136.699997 70.5) (width 0.2) (layer "B.Cu") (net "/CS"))
 (segment (start 178.5 73) (end 178.74 73) (width 0.2) (layer "F.Cu") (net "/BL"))
 (segment (start 178.74 73) (end 180.62 71.12) (width 0.2) (layer "F.Cu") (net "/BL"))
 (via (at 178.5 73) (size 0.6) (drill 0.3) (layers "F.Cu" "B.Cu") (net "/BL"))
 (segment (start 158.12 65.5) (end 158 65.5) (width 0.2) (layer "B.Cu") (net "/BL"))
 (segment (start 159 73) (end 178.5 73) (width 0.2) (layer "B.Cu") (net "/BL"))
 (segment (start 158.12 72.12) (end 159 73) (width 0.2) (layer "B.Cu") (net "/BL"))
 (segment (start 158.12 65.5) (end 158.12 72.12) (width 0.2) (layer "B.Cu") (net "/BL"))
 (via (at 165.38 71.12) (size 0.6) (drill 0.3) (layers "F.Cu" "B.Cu") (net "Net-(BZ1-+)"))
 (segment (start 204 62.8815) (end 197.088497 69.793003) (width 0.2) (layer "B.Cu") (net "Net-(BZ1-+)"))
 (segment (start 197.088497 69.793003) (end 166.706997 69.793003) (width 0.2) (layer "B.Cu") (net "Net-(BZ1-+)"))
 (segment (start 166.706997 69.793003) (end 165.38 71.12) (width 0.2) (layer "B.Cu") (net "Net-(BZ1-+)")))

